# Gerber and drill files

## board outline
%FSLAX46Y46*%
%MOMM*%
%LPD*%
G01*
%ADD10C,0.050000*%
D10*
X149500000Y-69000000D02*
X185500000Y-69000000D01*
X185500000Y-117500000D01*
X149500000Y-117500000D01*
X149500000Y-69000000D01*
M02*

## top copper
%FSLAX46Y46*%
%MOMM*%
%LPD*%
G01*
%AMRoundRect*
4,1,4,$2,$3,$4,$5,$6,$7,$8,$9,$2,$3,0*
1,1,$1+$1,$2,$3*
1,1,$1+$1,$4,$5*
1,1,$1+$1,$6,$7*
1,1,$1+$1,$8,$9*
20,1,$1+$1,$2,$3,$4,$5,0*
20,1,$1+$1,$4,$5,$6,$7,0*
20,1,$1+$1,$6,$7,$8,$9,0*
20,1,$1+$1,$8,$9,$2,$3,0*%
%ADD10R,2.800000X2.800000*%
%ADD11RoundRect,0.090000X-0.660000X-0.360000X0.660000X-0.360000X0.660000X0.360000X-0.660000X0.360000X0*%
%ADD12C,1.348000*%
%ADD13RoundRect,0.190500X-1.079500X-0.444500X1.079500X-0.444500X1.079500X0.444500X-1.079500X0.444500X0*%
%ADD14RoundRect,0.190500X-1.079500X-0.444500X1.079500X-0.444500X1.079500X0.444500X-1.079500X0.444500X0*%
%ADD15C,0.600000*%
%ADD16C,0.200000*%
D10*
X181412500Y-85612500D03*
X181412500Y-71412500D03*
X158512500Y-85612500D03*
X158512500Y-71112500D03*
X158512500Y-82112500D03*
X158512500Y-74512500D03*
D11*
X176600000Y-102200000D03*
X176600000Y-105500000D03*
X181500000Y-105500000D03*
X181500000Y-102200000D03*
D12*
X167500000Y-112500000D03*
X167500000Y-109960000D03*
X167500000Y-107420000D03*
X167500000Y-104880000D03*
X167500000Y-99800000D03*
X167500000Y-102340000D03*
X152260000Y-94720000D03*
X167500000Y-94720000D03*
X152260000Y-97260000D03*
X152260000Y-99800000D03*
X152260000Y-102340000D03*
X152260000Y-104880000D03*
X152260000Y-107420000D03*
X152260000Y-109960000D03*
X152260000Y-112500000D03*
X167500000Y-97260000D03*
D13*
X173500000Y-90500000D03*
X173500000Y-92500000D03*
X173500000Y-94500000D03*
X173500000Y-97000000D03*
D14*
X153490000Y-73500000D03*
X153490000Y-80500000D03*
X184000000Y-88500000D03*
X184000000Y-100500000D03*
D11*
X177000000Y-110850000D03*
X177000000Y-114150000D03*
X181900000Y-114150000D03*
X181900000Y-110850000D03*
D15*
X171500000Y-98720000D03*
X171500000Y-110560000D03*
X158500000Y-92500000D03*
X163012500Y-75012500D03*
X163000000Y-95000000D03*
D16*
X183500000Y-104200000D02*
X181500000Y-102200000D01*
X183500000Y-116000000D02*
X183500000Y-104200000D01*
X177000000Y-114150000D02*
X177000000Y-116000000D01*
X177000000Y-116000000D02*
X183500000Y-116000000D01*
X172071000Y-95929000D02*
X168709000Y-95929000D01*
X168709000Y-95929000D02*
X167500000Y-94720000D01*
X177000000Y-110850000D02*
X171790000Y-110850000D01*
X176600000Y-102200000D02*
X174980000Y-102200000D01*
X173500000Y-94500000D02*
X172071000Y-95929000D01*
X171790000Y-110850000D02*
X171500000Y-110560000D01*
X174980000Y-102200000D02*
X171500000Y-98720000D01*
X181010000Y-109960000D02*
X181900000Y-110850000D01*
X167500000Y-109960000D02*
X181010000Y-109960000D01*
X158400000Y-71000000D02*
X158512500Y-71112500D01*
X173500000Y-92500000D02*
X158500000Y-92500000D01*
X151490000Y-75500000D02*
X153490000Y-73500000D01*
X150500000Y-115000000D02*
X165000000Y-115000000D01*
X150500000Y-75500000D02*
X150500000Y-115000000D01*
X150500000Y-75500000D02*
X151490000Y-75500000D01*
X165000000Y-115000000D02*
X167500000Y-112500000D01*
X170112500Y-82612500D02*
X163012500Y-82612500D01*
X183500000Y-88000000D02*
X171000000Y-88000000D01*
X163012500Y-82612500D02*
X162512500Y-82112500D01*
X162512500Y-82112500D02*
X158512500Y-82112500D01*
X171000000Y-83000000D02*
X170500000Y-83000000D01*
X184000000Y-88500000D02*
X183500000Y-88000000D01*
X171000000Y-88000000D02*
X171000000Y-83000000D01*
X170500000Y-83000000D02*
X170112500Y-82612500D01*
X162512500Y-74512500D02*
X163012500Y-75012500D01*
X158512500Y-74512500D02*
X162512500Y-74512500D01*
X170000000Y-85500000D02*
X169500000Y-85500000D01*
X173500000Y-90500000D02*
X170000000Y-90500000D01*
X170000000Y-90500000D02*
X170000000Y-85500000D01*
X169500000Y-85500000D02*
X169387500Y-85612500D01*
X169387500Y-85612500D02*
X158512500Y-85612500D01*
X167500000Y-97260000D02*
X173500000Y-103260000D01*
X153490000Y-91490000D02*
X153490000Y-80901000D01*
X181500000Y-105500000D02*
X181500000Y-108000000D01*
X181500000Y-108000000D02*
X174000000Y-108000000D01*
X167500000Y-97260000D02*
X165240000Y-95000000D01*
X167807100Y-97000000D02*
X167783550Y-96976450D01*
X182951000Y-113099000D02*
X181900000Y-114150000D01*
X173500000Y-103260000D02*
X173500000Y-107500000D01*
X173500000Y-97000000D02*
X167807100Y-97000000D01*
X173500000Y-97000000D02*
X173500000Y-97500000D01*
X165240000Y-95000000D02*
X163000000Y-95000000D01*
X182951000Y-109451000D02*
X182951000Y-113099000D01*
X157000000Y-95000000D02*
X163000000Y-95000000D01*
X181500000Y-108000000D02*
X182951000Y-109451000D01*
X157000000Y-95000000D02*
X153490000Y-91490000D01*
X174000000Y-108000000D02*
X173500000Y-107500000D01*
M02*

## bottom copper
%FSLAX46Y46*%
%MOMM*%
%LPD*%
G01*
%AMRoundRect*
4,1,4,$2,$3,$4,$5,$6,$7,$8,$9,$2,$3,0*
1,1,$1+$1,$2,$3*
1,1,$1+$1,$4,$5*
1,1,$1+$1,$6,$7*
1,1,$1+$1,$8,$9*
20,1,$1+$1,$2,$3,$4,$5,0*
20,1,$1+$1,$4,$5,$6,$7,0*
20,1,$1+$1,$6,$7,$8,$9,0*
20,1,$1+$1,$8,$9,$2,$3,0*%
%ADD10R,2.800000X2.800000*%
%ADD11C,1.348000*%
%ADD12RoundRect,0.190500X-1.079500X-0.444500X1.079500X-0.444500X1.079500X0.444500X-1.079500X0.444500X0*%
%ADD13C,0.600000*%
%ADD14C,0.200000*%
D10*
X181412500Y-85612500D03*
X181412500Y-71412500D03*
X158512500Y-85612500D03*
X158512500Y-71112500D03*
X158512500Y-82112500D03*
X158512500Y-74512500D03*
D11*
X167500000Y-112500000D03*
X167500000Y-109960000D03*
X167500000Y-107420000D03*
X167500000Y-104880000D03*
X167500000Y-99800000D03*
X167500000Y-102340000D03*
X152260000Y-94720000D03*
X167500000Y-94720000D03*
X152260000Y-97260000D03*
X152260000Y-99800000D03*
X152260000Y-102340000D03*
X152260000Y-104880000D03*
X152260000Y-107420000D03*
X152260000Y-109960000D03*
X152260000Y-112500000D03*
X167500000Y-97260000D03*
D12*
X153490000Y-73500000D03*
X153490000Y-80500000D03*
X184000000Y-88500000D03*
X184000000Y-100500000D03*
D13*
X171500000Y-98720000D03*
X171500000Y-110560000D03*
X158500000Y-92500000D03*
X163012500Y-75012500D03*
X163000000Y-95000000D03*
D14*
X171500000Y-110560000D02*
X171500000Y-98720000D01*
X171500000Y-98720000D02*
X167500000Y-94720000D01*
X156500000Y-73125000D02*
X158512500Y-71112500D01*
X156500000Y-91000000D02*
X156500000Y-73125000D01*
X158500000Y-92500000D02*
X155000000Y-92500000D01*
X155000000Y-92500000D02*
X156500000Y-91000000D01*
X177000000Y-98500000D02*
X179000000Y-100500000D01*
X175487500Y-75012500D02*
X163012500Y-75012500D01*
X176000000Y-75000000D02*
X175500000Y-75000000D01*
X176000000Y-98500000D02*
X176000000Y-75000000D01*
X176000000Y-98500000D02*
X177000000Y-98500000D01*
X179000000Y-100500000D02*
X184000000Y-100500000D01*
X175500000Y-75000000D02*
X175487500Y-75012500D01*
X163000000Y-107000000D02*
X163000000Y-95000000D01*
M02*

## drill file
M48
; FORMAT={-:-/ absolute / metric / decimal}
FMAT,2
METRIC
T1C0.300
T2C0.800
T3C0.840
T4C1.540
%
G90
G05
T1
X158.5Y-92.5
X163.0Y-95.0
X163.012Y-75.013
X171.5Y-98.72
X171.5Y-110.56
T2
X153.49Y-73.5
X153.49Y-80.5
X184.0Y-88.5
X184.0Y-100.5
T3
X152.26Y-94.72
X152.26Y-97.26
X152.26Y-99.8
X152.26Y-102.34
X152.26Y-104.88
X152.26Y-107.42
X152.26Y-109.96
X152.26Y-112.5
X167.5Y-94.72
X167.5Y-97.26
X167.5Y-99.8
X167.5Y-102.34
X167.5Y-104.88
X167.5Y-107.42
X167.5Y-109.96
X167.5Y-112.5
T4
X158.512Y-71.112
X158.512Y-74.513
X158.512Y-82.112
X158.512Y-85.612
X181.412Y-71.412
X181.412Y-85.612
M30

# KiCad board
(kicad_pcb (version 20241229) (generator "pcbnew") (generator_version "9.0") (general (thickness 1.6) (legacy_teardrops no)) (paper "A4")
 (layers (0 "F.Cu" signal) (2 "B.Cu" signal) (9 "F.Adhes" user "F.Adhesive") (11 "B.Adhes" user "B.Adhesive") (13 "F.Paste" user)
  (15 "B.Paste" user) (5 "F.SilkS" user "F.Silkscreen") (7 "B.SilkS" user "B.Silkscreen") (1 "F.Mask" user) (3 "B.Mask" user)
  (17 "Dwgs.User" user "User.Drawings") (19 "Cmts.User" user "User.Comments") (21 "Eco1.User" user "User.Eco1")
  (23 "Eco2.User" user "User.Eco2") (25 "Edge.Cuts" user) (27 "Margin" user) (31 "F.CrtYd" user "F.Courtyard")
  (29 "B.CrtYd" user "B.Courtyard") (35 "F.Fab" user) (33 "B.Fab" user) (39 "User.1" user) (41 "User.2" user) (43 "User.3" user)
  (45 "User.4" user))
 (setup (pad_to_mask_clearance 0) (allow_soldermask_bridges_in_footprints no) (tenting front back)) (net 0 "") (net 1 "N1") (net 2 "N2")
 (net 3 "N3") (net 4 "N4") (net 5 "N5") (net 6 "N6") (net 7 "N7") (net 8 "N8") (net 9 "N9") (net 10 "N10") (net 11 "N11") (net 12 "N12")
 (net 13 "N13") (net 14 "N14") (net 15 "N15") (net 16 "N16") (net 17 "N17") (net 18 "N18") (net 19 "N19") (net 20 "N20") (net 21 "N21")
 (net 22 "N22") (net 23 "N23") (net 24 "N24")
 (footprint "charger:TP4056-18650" (layer "F.Cu") (at 183.1125 87.3125 180)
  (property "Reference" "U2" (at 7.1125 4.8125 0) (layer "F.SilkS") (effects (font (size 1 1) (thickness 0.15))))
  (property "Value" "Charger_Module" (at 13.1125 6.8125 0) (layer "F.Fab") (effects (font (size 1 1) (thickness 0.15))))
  (pad "1" thru_hole rect (at 1.7 1.7 180) (size 2.8 2.8) (drill 1.54) (layers "*.Cu" "*.Mask") (remove_unused_layers no) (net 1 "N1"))
  (pad "2" thru_hole rect (at 1.7 15.9 180) (size 2.8 2.8) (drill 1.54) (layers "*.Cu" "*.Mask") (remove_unused_layers no) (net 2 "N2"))
  (pad "3" thru_hole rect (at 24.6 1.7 180) (size 2.8 2.8) (drill 1.54) (layers "*.Cu" "*.Mask") (remove_unused_layers no) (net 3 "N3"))
  (pad "4" thru_hole rect (at 24.6 16.2 180) (size 2.8 2.8) (drill 1.54) (layers "*.Cu" "*.Mask") (remove_unused_layers no) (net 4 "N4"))
  (pad "5" thru_hole rect (at 24.6 5.2 180) (size 2.8 2.8) (drill 1.54) (layers "*.Cu" "*.Mask") (remove_unused_layers no) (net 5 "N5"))
  (pad "6" thru_hole rect (at 24.6 12.8 180) (size 2.8 2.8) (drill 1.54) (layers "*.Cu" "*.Mask") (remove_unused_layers no) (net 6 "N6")))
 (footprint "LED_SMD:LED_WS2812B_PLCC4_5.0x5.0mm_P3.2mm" (layer "F.Cu") (at 179.05 103.85)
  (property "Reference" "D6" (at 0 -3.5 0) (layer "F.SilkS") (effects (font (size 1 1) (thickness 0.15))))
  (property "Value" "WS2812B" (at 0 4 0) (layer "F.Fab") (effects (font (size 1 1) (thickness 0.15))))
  (pad "1" smd roundrect (at -2.45 -1.65) (size 1.5 0.9) (layers "F.Cu" "F.Mask" "F.Paste") (roundrect_rratio 0.1) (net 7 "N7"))
  (pad "2" smd roundrect (at -2.45 1.65) (size 1.5 0.9) (layers "F.Cu" "F.Mask" "F.Paste") (roundrect_rratio 0.1) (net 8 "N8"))
  (pad "3" smd roundrect (at 2.45 1.65) (size 1.5 0.9) (layers "F.Cu" "F.Mask" "F.Paste") (roundrect_rratio 0.1) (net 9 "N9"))
  (pad "4" smd roundrect (at 2.45 -1.65) (size 1.5 0.9) (layers "F.Cu" "F.Mask" "F.Paste") (roundrect_rratio 0.1) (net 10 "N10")))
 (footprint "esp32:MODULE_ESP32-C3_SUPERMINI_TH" (layer "F.Cu") (at 159.88 104.62)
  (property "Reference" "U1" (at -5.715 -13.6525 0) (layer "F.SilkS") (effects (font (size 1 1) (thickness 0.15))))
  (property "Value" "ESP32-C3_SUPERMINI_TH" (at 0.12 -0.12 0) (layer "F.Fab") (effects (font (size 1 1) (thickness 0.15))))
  (pad "0" thru_hole circle (at 7.62 7.88) (size 1.348 1.348) (drill 0.84) (layers "*.Cu" "*.Mask") (remove_unused_layers no) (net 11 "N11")
   (solder_mask_margin 0.102))
  (pad "1" thru_hole circle (at 7.62 5.34) (size 1.348 1.348) (drill 0.84) (layers "*.Cu" "*.Mask") (remove_unused_layers no) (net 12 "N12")
   (solder_mask_margin 0.102))
  (pad "2" thru_hole circle (at 7.62 2.8) (size 1.348 1.348) (drill 0.84) (layers "*.Cu" "*.Mask") (remove_unused_layers no) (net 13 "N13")
   (solder_mask_margin 0.102))
  (pad "3" thru_hole circle (at 7.62 0.26) (size 1.348 1.348) (drill 0.84) (layers "*.Cu" "*.Mask") (remove_unused_layers no) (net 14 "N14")
   (solder_mask_margin 0.102))
  (pad "3.3" thru_hole circle (at 7.62 -4.82) (size 1.348 1.348) (drill 0.84) (layers "*.Cu" "*.Mask") (remove_unused_layers no)
   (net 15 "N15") (solder_mask_margin 0.102))
  (pad "4" thru_hole circle (at 7.62 -2.28) (size 1.348 1.348) (drill 0.84) (layers "*.Cu" "*.Mask") (remove_unused_layers no)
   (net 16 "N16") (solder_mask_margin 0.102))
  (pad "5" thru_hole circle (at -7.62 -9.9) (size 1.348 1.348) (drill 0.84) (layers "*.Cu" "*.Mask") (remove_unused_layers no)
   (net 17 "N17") (solder_mask_margin 0.102))
  (pad "5V" thru_hole circle (at 7.62 -9.9) (size 1.348 1.348) (drill 0.84) (layers "*.Cu" "*.Mask") (remove_unused_layers no) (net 7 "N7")
   (solder_mask_margin 0.102))
  (pad "6" thru_hole circle (at -7.62 -7.36) (size 1.348 1.348) (drill 0.84) (layers "*.Cu" "*.Mask") (remove_unused_layers no)
   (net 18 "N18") (solder_mask_margin 0.102))
  (pad "7" thru_hole circle (at -7.62 -4.82) (size 1.348 1.348) (drill 0.84) (layers "*.Cu" "*.Mask") (remove_unused_layers no)
   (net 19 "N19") (solder_mask_margin 0.102))
  (pad "8" thru_hole circle (at -7.62 -2.28) (size 1.348 1.348) (drill 0.84) (layers "*.Cu" "*.Mask") (remove_unused_layers no)
   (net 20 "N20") (solder_mask_margin 0.102))
  (pad "9" thru_hole circle (at -7.62 0.26) (size 1.348 1.348) (drill 0.84) (layers "*.Cu" "*.Mask") (remove_unused_layers no)
   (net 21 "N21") (solder_mask_margin 0.102))
  (pad "10" thru_hole circle (at -7.62 2.8) (size 1.348 1.348) (drill 0.84) (layers "*.Cu" "*.Mask") (remove_unused_layers no)
   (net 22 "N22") (solder_mask_margin 0.102))
  (pad "20" thru_hole circle (at -7.62 5.34) (size 1.348 1.348) (drill 0.84) (layers "*.Cu" "*.Mask") (remove_unused_layers no)
   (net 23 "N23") (solder_mask_margin 0.102))
  (pad "21" thru_hole circle (at -7.62 7.88) (size 1.348 1.348) (drill 0.84) (layers "*.Cu" "*.Mask") (remove_unused_layers no)
   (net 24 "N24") (solder_mask_margin 0.102))
  (pad "G" thru_hole circle (at 7.62 -7.36) (size 1.348 1.348) (drill 0.84) (layers "*.Cu" "*.Mask") (remove_unused_layers no) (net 9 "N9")
   (solder_mask_margin 0.102)))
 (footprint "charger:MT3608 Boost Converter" (layer "F.Cu") (at 178 92)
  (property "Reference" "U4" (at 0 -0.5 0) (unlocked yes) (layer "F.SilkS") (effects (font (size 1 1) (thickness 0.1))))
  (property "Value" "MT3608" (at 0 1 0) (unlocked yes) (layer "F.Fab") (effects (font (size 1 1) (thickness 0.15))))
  (pad "1" connect roundrect (at -4.5 -1.5) (size 2.54 1.27) (layers "F.Cu" "F.Mask") (roundrect_rratio 0.15) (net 3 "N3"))
  (pad "2" connect roundrect (at -4.5 0.5) (size 2.54 1.27) (layers "F.Cu" "F.Mask") (roundrect_rratio 0.15) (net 4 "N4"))
  (pad "3" connect roundrect (at -4.5 2.5) (size 2.54 1.27) (layers "F.Cu" "F.Mask") (roundrect_rratio 0.15) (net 7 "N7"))
  (pad "4" connect roundrect (at -4.5 5) (size 2.54 1.27) (layers "F.Cu" "F.Mask") (roundrect_rratio 0.15) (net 9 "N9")))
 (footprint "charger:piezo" (layer "F.Cu") (at 147.49 77)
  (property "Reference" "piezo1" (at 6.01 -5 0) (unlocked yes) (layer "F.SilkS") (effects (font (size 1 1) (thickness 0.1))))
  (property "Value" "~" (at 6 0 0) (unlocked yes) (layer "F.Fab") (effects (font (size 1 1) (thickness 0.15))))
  (pad "1" thru_hole roundrect (at 6 -3.5) (size 2.54 1.27) (drill 0.8) (layers "*.Cu" "*.Mask") (remove_unused_layers no)
   (roundrect_rratio 0.15) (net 11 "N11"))
  (pad "2" thru_hole roundrect (at 6 3.5) (size 2.54 1.27) (drill 0.8) (layers "*.Cu" "*.Mask") (remove_unused_layers no)
   (roundrect_rratio 0.15) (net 9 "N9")))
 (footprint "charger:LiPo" (layer "F.Cu") (at 168.5 94.5)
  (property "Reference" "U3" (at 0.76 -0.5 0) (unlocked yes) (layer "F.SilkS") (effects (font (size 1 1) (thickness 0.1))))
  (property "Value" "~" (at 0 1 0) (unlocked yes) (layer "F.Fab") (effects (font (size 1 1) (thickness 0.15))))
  (pad "1" thru_hole roundrect (at 15.5 -6) (size 2.54 1.27) (drill 0.8) (layers "*.Cu" "*.Mask") (remove_unused_layers no)
   (roundrect_rratio 0.15) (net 5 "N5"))
  (pad "2" thru_hole roundrect (at 15.5 6) (size 2.54 1.27) (drill 0.8) (layers "*.Cu" "*.Mask") (remove_unused_layers no)
   (roundrect_rratio 0.15) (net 6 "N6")))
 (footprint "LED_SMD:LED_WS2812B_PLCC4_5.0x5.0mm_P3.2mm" (layer "F.Cu") (at 179.45 112.5)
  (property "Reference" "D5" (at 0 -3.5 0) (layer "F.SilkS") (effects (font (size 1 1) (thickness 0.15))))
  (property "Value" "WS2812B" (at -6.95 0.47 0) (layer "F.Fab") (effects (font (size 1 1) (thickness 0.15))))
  (pad "1" smd roundrect (at -2.45 -1.65) (size 1.5 0.9) (layers "F.Cu" "F.Mask" "F.Paste") (roundrect_rratio 0.1) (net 7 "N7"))
  (pad "2" smd roundrect (at -2.45 1.65) (size 1.5 0.9) (layers "F.Cu" "F.Mask" "F.Paste") (roundrect_rratio 0.1) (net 10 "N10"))
  (pad "3" smd roundrect (at 2.45 1.65) (size 1.5 0.9) (layers "F.Cu" "F.Mask" "F.Paste") (roundrect_rratio 0.1) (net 9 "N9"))
  (pad "4" smd roundrect (at 2.45 -1.65) (size 1.5 0.9) (layers "F.Cu" "F.Mask" "F.Paste") (roundrect_rratio 0.1) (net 12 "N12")))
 (gr_rect (start 149.5 69) (end 185.5 117.5) (stroke (width 0.05) (type default)) (fill no) (layer "Edge.Cuts"))
 (segment (start 183.5 104.2) (end 181.5 102.2) (width 0.2) (layer "F.Cu") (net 10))
 (segment (start 183.5 116) (end 183.5 104.2) (width 0.2) (layer "F.Cu") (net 10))
 (segment (start 177 114.15) (end 177 116) (width 0.2) (layer "F.Cu") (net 10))
 (segment (start 177 116) (end 183.5 116) (width 0.2) (layer "F.Cu") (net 10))
 (segment (start 172.071 95.929) (end 168.709 95.929) (width 0.2) (layer "F.Cu") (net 7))
 (segment (start 168.709 95.929) (end 167.5 94.72) (width 0.2) (layer "F.Cu") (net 7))
 (segment (start 177 110.85) (end 171.79 110.85) (width 0.2) (layer "F.Cu") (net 7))
 (segment (start 176.6 102.2) (end 174.98 102.2) (width 0.2) (layer "F.Cu") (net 7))
 (segment (start 173.5 94.5) (end 172.071 95.929) (width 0.2) (layer "F.Cu") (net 7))
 (segment (start 171.79 110.85) (end 171.5 110.56) (width 0.2) (layer "F.Cu") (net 7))
 (segment (start 174.98 102.2) (end 171.5 98.72) (width 0.2) (layer "F.Cu") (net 7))
 (via (at 171.5 98.72) (size 0.6) (drill 0.3) (layers "F.Cu" "B.Cu") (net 7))
 (via (at 171.5 110.56) (size 0.6) (drill 0.3) (layers "F.Cu" "B.Cu") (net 7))
 (segment (start 171.5 110.56) (end 171.5 98.72) (width 0.2) (layer "B.Cu") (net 7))
 (segment (start 171.5 98.72) (end 167.5 94.72) (width 0.2) (layer "B.Cu") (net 7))
 (segment (start 181.01 109.96) (end 181.9 110.85) (width 0.2) (layer "F.Cu") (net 12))
 (segment (start 167.5 109.96) (end 181.01 109.96) (width 0.2) (layer "F.Cu") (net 12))
 (segment (start 158.4 71) (end 158.5125 71.1125) (width 0.2) (layer "F.Cu") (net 4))
 (segment (start 173.5 92.5) (end 158.5 92.5) (width 0.2) (layer "F.Cu") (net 4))
 (via (at 158.5 92.5) (size 0.6) (drill 0.3) (layers "F.Cu" "B.Cu") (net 4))
 (segment (start 156.5 73.125) (end 158.5125 71.1125) (width 0.2) (layer "B.Cu") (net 4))
 (segment (start 156.5 91) (end 156.5 73.125) (width 0.2) (layer "B.Cu") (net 4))
 (segment (start 158.5 92.5) (end 155 92.5) (width 0.2) (layer "B.Cu") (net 4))
 (segment (start 155 92.5) (end 156.5 91) (width 0.2) (layer "B.Cu") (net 4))
 (segment (start 151.49 75.5) (end 153.49 73.5) (width 0.2) (layer "F.Cu") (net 11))
 (segment (start 150.5 115) (end 165 115) (width 0.2) (layer "F.Cu") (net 11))
 (segment (start 150.5 75.5) (end 150.5 115) (width 0.2) (layer "F.Cu") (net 11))
 (segment (start 150.5 75.5) (end 151.49 75.5) (width 0.2) (layer "F.Cu") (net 11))
 (segment (start 165 115) (end 167.5 112.5) (width 0.2) (layer "F.Cu") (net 11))
 (segment (start 170.1125 82.6125) (end 163.0125 82.6125) (width 0.2) (layer "F.Cu") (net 5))
 (segment (start 183.5 88) (end 171 88) (width 0.2) (layer "F.Cu") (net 5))
 (segment (start 163.0125 82.6125) (end 162.5125 82.1125) (width 0.2) (layer "F.Cu") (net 5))
 (segment (start 162.5125 82.1125) (end 158.5125 82.1125) (width 0.2) (layer "F.Cu") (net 5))
 (segment (start 171 83) (end 170.5 83) (width 0.2) (layer "F.Cu") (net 5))
 (segment (start 184 88.5) (end 183.5 88) (width 0.2) (layer "F.Cu") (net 5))
 (segment (start 171 88) (end 171 83) (width 0.2) (layer "F.Cu") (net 5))
 (segment (start 170.5 83) (end 170.1125 82.6125) (width 0.2) (layer "F.Cu") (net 5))
 (segment (start 162.5125 74.5125) (end 163.0125 75.0125) (width 0.2) (layer "F.Cu") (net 6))
 (segment (start 158.5125 74.5125) (end 162.5125 74.5125) (width 0.2) (layer "F.Cu") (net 6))
 (via (at 163.0125 75.0125) (size 0.6) (drill 0.3) (layers "F.Cu" "B.Cu") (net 6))
 (segment (start 177 98.5) (end 179 100.5) (width 0.2) (layer "B.Cu") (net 6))
 (segment (start 175.4875 75.0125) (end 163.0125 75.0125) (width 0.2) (layer "B.Cu") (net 6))
 (segment (start 176 75) (end 175.5 75) (width 0.2) (layer "B.Cu") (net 6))
 (segment (start 176 98.5) (end 176 75) (width 0.2) (layer "B.Cu") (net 6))
 (segment (start 176 98.5) (end 177 98.5) (width 0.2) (layer "B.Cu") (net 6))
 (segment (start 179 100.5) (end 184 100.5) (width 0.2) (layer "B.Cu") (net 6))
 (segment (start 175.5 75) (end 175.4875 75.0125) (width 0.2) (layer "B.Cu") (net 6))
 (segment (start 170 85.5) (end 169.5 85.5) (width 0.2) (layer "F.Cu") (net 3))
 (segment (start 173.5 90.5) (end 170 90.5) (width 0.2) (layer "F.Cu") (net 3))
 (segment (start 170 90.5) (end 170 85.5) (width 0.2) (layer "F.Cu") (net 3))
 (segment (start 169.5 85.5) (end 169.3875 85.6125) (width 0.2) (layer "F.Cu") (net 3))
 (segment (start 169.3875 85.6125) (end 158.5125 85.6125) (width 0.2) (layer "F.Cu") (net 3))
 (segment (start 167.5 97.26) (end 173.5 103.26) (width 0.2) (layer "F.Cu") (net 9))
 (segment (start 153.49 91.49) (end 153.49 80.901) (width 0.2) (layer "F.Cu") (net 9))
 (segment (start 181.5 105.5) (end 181.5 108) (width 0.2) (layer "F.Cu") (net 9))
 (segment (start 181.5 108) (end 174 108) (width 0.2) (layer "F.Cu") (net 9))
 (segment (start 167.5 97.26) (end 165.24 95) (width 0.2) (layer "F.Cu") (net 9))
 (segment (start 167.8071 97) (end 167.78355 96.97645) (width 0.2) (layer "F.Cu") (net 9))
 (segment (start 182.951 113.099) (end 181.9 114.15) (width 0.2) (layer "F.Cu") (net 9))
 (segment (start 173.5 103.26) (end 173.5 107.5) (width 0.2) (layer "F.Cu") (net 9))
 (segment (start 173.5 97) (end 167.8071 97) (width 0.2) (layer "F.Cu") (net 9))
 (segment (start 173.5 97) (end 173.5 97.5) (width 0.2) (layer "F.Cu") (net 9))
 (segment (start 165.24 95) (end 163 95) (width 0.2) (layer "F.Cu") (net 9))
 (segment (start 182.951 109.451) (end 182.951 113.099) (width 0.2) (layer "F.Cu") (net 9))
 (segment (start 157 95) (end 163 95) (width 0.2) (layer "F.Cu") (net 9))
 (segment (start 181.5 108) (end 182.951 109.451) (width 0.2) (layer "F.Cu") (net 9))
 (segment (start 157 95) (end 153.49 91.49) (width 0.2) (layer "F.Cu") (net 9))
 (segment (start 174 108) (end 173.5 107.5) (width 0.2) (layer "F.Cu") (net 9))
 (via (at 163 95) (size 0.6) (drill 0.3) (layers "F.Cu" "B.Cu") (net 9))
 (segment (start 163 107) (end 163 95) (width 0.2) (layer "B.Cu") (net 9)))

